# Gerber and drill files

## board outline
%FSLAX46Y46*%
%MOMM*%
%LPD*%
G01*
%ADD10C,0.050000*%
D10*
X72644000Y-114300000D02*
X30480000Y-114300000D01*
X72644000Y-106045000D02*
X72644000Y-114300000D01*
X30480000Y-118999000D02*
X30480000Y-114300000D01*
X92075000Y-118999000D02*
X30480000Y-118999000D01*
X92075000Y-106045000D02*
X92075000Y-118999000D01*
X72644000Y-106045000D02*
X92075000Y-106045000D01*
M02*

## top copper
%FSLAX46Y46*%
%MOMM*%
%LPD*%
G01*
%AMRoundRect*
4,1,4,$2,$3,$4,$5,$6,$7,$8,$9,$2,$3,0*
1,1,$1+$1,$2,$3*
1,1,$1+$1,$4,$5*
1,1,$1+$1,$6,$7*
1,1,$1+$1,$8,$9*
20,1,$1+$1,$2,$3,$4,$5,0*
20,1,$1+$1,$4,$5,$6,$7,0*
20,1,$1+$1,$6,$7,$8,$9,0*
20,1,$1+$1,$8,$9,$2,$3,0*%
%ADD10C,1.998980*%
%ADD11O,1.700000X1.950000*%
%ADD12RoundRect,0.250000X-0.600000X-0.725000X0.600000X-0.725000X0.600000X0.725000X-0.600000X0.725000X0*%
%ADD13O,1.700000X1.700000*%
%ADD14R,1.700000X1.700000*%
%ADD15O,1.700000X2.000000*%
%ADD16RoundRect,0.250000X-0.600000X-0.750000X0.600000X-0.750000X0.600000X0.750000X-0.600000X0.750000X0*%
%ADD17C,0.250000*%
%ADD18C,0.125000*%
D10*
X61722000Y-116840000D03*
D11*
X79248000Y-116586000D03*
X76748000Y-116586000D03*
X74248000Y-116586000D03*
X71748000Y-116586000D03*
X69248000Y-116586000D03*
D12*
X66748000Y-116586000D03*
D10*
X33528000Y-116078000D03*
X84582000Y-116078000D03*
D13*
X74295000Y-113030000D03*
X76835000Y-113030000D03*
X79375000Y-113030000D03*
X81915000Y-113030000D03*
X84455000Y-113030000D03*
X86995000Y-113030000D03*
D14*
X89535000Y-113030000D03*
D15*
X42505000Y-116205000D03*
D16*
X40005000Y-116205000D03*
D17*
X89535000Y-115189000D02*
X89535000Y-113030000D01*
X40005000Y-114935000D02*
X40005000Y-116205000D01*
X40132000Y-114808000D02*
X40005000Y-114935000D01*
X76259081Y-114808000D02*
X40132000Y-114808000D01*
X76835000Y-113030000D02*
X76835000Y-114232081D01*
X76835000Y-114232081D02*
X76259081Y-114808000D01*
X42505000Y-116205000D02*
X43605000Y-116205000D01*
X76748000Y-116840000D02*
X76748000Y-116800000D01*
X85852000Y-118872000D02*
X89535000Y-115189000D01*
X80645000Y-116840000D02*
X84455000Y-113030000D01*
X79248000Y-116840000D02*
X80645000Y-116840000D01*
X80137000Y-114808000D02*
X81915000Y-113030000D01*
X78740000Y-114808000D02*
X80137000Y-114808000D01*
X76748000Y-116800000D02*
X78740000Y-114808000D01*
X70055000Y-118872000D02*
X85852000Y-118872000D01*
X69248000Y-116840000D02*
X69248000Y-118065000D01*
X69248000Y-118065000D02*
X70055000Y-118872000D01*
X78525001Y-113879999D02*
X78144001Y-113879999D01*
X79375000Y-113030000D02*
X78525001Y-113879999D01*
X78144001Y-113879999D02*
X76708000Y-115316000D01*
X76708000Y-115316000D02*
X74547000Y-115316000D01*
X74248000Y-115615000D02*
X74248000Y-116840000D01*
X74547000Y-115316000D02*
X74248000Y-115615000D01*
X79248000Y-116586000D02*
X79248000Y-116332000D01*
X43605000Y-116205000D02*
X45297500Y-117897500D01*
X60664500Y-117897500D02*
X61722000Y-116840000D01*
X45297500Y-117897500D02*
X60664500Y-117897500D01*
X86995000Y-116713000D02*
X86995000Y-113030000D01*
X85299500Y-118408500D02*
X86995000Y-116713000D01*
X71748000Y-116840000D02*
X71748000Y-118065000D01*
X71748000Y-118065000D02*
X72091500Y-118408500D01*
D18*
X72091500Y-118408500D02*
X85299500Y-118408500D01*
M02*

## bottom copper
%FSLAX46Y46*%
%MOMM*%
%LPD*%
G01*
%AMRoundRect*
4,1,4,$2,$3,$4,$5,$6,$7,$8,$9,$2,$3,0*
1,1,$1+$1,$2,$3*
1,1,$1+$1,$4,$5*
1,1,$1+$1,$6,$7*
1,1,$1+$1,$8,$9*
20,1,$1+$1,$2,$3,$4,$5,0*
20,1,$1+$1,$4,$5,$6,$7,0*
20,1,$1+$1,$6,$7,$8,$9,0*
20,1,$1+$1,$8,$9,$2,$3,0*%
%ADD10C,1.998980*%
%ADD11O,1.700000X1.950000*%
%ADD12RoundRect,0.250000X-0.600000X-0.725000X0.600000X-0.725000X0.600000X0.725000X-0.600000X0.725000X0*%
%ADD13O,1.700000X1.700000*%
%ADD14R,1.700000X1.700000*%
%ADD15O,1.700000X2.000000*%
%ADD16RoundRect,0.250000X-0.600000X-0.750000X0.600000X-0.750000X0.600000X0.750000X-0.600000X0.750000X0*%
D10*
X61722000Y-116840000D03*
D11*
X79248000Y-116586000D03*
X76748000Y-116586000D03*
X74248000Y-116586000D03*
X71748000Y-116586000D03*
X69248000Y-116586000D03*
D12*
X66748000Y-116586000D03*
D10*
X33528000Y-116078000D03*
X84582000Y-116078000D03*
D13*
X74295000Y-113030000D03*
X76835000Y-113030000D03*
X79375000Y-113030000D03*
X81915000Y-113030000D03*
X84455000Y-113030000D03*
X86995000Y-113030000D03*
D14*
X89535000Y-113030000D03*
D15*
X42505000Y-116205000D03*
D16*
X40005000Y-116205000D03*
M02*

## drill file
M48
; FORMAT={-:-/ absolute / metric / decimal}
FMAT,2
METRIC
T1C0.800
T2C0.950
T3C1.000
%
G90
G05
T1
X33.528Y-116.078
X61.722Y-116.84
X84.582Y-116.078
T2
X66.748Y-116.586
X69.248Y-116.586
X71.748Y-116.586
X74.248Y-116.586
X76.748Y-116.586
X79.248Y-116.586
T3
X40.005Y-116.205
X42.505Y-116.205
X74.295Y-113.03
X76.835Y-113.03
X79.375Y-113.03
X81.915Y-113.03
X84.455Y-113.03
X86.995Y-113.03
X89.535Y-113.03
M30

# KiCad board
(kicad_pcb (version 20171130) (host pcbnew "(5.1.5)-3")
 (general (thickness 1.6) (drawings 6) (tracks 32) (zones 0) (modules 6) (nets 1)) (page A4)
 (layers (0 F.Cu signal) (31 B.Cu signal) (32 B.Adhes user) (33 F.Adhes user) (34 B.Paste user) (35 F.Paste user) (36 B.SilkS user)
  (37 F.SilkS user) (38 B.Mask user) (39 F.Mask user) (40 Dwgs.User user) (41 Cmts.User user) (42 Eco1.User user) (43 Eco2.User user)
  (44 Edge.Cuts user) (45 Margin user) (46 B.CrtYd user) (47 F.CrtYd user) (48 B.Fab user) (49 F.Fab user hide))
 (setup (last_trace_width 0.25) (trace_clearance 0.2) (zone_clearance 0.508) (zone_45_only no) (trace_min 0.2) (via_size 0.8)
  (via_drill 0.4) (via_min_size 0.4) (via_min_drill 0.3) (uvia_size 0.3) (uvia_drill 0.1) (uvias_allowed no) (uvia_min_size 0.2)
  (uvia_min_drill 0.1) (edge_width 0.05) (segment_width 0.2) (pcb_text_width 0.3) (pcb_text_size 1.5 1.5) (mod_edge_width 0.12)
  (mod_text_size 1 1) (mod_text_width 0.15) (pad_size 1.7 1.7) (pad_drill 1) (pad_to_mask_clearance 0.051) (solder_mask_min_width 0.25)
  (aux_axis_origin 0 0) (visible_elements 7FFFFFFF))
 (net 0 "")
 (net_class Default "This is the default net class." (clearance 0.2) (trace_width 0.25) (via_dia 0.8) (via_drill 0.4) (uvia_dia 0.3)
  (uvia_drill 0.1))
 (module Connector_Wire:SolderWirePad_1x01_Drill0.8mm (layer F.Cu) (at 61.722 116.84)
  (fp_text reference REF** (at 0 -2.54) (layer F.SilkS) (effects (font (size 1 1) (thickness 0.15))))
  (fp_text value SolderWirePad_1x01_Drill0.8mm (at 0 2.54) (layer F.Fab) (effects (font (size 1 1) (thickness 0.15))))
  (pad 1 thru_hole circle (at 0 0) (size 1.99898 1.99898) (drill 0.8001) (layers *.Cu *.Mask)))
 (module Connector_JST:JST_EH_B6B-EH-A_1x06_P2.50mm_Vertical (layer F.Cu) (at 66.748 116.586)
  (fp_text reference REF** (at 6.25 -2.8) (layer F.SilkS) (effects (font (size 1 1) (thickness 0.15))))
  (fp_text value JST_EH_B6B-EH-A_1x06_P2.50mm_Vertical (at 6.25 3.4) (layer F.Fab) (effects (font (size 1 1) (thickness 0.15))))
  (pad 6 thru_hole oval (at 12.5 0) (size 1.7 1.95) (drill 0.95) (layers *.Cu *.Mask))
  (pad 5 thru_hole oval (at 10 0) (size 1.7 1.95) (drill 0.95) (layers *.Cu *.Mask))
  (pad 4 thru_hole oval (at 7.5 0) (size 1.7 1.95) (drill 0.95) (layers *.Cu *.Mask))
  (pad 3 thru_hole oval (at 5 0) (size 1.7 1.95) (drill 0.95) (layers *.Cu *.Mask))
  (pad 2 thru_hole oval (at 2.5 0) (size 1.7 1.95) (drill 0.95) (layers *.Cu *.Mask))
  (pad 1 thru_hole roundrect (at 0 0) (size 1.7 1.95) (drill 0.95) (layers *.Cu *.Mask) (roundrect_rratio 0.147059)))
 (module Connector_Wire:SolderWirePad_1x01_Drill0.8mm (layer F.Cu) (at 33.528 116.078)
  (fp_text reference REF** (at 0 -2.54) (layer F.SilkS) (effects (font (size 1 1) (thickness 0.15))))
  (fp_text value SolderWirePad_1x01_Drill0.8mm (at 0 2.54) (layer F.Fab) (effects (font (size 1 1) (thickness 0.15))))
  (pad 1 thru_hole circle (at 0 0) (size 1.99898 1.99898) (drill 0.8001) (layers *.Cu *.Mask)))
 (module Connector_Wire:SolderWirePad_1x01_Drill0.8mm (layer F.Cu) (at 84.582 116.078)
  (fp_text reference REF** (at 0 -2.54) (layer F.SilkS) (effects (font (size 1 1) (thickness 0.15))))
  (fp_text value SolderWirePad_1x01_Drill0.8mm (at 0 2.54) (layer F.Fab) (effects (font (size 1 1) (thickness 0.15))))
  (pad 1 thru_hole circle (at 0 0) (size 1.99898 1.99898) (drill 0.8001) (layers *.Cu *.Mask)))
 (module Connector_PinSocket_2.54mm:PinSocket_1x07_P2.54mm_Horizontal (layer F.Cu) (at 89.535 113.03 270)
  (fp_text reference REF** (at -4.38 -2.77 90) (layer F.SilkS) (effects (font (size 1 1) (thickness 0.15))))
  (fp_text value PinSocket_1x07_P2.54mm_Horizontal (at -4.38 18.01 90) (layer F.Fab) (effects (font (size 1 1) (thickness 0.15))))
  (pad 5v thru_hole oval (at 0 15.24 270) (size 1.7 1.7) (drill 1) (layers *.Cu *.Mask))
  (pad in1 thru_hole oval (at 0 12.7 270) (size 1.7 1.7) (drill 1) (layers *.Cu *.Mask))
  (pad in2 thru_hole oval (at 0 10.16 270) (size 1.7 1.7) (drill 1) (layers *.Cu *.Mask))
  (pad in3 thru_hole oval (at 0 7.62 270) (size 1.7 1.7) (drill 1) (layers *.Cu *.Mask))
  (pad mot1 thru_hole oval (at 0 5.08 270) (size 1.7 1.7) (drill 1) (layers *.Cu *.Mask))
  (pad gnd thru_hole oval (at 0 2.54 270) (size 1.7 1.7) (drill 1) (layers *.Cu *.Mask))
  (pad mot2 thru_hole rect (at 0 0 270) (size 1.7 1.7) (drill 1) (layers *.Cu *.Mask)))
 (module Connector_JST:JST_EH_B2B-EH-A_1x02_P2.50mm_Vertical (layer F.Cu) (at 40.005 116.205)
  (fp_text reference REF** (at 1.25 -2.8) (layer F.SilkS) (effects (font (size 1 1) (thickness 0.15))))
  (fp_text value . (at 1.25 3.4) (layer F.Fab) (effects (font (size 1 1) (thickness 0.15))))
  (pad 2 thru_hole oval (at 2.5 0) (size 1.7 2) (drill 1) (layers *.Cu *.Mask))
  (pad 1 thru_hole roundrect (at 0 0) (size 1.7 2) (drill 1) (layers *.Cu *.Mask) (roundrect_rratio 0.147059)))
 (gr_line (start 72.644 114.3) (end 30.48 114.3) (layer Edge.Cuts) (width 0.05))
 (gr_line (start 72.644 106.045) (end 72.644 114.3) (layer Edge.Cuts) (width 0.05))
 (gr_line (start 30.48 118.999) (end 30.48 114.3) (layer Edge.Cuts) (width 0.05))
 (gr_line (start 92.075 118.999) (end 30.48 118.999) (layer Edge.Cuts) (width 0.05))
 (gr_line (start 92.075 106.045) (end 92.075 118.999) (layer Edge.Cuts) (width 0.05))
 (gr_line (start 72.644 106.045) (end 92.075 106.045) (layer Edge.Cuts) (width 0.05))
 (segment (start 89.535 115.189) (end 89.535 113.03) (width 0.25) (layer F.Cu) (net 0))
 (segment (start 40.005 114.935) (end 40.005 116.205) (width 0.25) (layer F.Cu) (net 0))
 (segment (start 40.132 114.808) (end 40.005 114.935) (width 0.25) (layer F.Cu) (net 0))
 (segment (start 76.259081 114.808) (end 40.132 114.808) (width 0.25) (layer F.Cu) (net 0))
 (segment (start 76.835 113.03) (end 76.835 114.232081) (width 0.25) (layer F.Cu) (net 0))
 (segment (start 76.835 114.232081) (end 76.259081 114.808) (width 0.25) (layer F.Cu) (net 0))
 (segment (start 42.505 116.205) (end 43.605 116.205) (width 0.25) (layer F.Cu) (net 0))
 (segment (start 76.748 116.84) (end 76.748 116.8) (width 0.25) (layer F.Cu) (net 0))
 (segment (start 85.852 118.872) (end 89.535 115.189) (width 0.25) (layer F.Cu) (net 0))
 (segment (start 80.645 116.84) (end 84.455 113.03) (width 0.25) (layer F.Cu) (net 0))
 (segment (start 79.248 116.84) (end 80.645 116.84) (width 0.25) (layer F.Cu) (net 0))
 (segment (start 80.137 114.808) (end 81.915 113.03) (width 0.25) (layer F.Cu) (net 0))
 (segment (start 78.74 114.808) (end 80.137 114.808) (width 0.25) (layer F.Cu) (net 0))
 (segment (start 76.748 116.8) (end 78.74 114.808) (width 0.25) (layer F.Cu) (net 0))
 (segment (start 70.055 118.872) (end 85.852 118.872) (width 0.25) (layer F.Cu) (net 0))
 (segment (start 69.248 116.84) (end 69.248 118.065) (width 0.25) (layer F.Cu) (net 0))
 (segment (start 69.248 118.065) (end 70.055 118.872) (width 0.25) (layer F.Cu) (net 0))
 (segment (start 78.525001 113.879999) (end 78.144001 113.879999) (width 0.25) (layer F.Cu) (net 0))
 (segment (start 79.375 113.03) (end 78.525001 113.879999) (width 0.25) (layer F.Cu) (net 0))
 (segment (start 78.144001 113.879999) (end 76.708 115.316) (width 0.25) (layer F.Cu) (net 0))
 (segment (start 76.708 115.316) (end 74.547 115.316) (width 0.25) (layer F.Cu) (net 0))
 (segment (start 74.248 115.615) (end 74.248 116.84) (width 0.25) (layer F.Cu) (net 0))
 (segment (start 74.547 115.316) (end 74.248 115.615) (width 0.25) (layer F.Cu) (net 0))
 (segment (start 79.248 116.586) (end 79.248 116.332) (width 0.25) (layer F.Cu) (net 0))
 (segment (start 43.605 116.205) (end 45.2975 117.8975) (width 0.25) (layer F.Cu) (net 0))
 (segment (start 60.6645 117.8975) (end 61.722 116.84) (width 0.25) (layer F.Cu) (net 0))
 (segment (start 45.2975 117.8975) (end 60.6645 117.8975) (width 0.25) (layer F.Cu) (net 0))
 (segment (start 86.995 116.713) (end 86.995 113.03) (width 0.25) (layer F.Cu) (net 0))
 (segment (start 85.2995 118.4085) (end 86.995 116.713) (width 0.25) (layer F.Cu) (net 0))
 (segment (start 71.748 116.84) (end 71.748 118.065) (width 0.25) (layer F.Cu) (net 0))
 (segment (start 71.748 118.065) (end 72.0915 118.4085) (width 0.25) (layer F.Cu) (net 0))
 (segment (start 72.0915 118.4085) (end 85.2995 118.4085) (width 0.125) (layer F.Cu) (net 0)))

